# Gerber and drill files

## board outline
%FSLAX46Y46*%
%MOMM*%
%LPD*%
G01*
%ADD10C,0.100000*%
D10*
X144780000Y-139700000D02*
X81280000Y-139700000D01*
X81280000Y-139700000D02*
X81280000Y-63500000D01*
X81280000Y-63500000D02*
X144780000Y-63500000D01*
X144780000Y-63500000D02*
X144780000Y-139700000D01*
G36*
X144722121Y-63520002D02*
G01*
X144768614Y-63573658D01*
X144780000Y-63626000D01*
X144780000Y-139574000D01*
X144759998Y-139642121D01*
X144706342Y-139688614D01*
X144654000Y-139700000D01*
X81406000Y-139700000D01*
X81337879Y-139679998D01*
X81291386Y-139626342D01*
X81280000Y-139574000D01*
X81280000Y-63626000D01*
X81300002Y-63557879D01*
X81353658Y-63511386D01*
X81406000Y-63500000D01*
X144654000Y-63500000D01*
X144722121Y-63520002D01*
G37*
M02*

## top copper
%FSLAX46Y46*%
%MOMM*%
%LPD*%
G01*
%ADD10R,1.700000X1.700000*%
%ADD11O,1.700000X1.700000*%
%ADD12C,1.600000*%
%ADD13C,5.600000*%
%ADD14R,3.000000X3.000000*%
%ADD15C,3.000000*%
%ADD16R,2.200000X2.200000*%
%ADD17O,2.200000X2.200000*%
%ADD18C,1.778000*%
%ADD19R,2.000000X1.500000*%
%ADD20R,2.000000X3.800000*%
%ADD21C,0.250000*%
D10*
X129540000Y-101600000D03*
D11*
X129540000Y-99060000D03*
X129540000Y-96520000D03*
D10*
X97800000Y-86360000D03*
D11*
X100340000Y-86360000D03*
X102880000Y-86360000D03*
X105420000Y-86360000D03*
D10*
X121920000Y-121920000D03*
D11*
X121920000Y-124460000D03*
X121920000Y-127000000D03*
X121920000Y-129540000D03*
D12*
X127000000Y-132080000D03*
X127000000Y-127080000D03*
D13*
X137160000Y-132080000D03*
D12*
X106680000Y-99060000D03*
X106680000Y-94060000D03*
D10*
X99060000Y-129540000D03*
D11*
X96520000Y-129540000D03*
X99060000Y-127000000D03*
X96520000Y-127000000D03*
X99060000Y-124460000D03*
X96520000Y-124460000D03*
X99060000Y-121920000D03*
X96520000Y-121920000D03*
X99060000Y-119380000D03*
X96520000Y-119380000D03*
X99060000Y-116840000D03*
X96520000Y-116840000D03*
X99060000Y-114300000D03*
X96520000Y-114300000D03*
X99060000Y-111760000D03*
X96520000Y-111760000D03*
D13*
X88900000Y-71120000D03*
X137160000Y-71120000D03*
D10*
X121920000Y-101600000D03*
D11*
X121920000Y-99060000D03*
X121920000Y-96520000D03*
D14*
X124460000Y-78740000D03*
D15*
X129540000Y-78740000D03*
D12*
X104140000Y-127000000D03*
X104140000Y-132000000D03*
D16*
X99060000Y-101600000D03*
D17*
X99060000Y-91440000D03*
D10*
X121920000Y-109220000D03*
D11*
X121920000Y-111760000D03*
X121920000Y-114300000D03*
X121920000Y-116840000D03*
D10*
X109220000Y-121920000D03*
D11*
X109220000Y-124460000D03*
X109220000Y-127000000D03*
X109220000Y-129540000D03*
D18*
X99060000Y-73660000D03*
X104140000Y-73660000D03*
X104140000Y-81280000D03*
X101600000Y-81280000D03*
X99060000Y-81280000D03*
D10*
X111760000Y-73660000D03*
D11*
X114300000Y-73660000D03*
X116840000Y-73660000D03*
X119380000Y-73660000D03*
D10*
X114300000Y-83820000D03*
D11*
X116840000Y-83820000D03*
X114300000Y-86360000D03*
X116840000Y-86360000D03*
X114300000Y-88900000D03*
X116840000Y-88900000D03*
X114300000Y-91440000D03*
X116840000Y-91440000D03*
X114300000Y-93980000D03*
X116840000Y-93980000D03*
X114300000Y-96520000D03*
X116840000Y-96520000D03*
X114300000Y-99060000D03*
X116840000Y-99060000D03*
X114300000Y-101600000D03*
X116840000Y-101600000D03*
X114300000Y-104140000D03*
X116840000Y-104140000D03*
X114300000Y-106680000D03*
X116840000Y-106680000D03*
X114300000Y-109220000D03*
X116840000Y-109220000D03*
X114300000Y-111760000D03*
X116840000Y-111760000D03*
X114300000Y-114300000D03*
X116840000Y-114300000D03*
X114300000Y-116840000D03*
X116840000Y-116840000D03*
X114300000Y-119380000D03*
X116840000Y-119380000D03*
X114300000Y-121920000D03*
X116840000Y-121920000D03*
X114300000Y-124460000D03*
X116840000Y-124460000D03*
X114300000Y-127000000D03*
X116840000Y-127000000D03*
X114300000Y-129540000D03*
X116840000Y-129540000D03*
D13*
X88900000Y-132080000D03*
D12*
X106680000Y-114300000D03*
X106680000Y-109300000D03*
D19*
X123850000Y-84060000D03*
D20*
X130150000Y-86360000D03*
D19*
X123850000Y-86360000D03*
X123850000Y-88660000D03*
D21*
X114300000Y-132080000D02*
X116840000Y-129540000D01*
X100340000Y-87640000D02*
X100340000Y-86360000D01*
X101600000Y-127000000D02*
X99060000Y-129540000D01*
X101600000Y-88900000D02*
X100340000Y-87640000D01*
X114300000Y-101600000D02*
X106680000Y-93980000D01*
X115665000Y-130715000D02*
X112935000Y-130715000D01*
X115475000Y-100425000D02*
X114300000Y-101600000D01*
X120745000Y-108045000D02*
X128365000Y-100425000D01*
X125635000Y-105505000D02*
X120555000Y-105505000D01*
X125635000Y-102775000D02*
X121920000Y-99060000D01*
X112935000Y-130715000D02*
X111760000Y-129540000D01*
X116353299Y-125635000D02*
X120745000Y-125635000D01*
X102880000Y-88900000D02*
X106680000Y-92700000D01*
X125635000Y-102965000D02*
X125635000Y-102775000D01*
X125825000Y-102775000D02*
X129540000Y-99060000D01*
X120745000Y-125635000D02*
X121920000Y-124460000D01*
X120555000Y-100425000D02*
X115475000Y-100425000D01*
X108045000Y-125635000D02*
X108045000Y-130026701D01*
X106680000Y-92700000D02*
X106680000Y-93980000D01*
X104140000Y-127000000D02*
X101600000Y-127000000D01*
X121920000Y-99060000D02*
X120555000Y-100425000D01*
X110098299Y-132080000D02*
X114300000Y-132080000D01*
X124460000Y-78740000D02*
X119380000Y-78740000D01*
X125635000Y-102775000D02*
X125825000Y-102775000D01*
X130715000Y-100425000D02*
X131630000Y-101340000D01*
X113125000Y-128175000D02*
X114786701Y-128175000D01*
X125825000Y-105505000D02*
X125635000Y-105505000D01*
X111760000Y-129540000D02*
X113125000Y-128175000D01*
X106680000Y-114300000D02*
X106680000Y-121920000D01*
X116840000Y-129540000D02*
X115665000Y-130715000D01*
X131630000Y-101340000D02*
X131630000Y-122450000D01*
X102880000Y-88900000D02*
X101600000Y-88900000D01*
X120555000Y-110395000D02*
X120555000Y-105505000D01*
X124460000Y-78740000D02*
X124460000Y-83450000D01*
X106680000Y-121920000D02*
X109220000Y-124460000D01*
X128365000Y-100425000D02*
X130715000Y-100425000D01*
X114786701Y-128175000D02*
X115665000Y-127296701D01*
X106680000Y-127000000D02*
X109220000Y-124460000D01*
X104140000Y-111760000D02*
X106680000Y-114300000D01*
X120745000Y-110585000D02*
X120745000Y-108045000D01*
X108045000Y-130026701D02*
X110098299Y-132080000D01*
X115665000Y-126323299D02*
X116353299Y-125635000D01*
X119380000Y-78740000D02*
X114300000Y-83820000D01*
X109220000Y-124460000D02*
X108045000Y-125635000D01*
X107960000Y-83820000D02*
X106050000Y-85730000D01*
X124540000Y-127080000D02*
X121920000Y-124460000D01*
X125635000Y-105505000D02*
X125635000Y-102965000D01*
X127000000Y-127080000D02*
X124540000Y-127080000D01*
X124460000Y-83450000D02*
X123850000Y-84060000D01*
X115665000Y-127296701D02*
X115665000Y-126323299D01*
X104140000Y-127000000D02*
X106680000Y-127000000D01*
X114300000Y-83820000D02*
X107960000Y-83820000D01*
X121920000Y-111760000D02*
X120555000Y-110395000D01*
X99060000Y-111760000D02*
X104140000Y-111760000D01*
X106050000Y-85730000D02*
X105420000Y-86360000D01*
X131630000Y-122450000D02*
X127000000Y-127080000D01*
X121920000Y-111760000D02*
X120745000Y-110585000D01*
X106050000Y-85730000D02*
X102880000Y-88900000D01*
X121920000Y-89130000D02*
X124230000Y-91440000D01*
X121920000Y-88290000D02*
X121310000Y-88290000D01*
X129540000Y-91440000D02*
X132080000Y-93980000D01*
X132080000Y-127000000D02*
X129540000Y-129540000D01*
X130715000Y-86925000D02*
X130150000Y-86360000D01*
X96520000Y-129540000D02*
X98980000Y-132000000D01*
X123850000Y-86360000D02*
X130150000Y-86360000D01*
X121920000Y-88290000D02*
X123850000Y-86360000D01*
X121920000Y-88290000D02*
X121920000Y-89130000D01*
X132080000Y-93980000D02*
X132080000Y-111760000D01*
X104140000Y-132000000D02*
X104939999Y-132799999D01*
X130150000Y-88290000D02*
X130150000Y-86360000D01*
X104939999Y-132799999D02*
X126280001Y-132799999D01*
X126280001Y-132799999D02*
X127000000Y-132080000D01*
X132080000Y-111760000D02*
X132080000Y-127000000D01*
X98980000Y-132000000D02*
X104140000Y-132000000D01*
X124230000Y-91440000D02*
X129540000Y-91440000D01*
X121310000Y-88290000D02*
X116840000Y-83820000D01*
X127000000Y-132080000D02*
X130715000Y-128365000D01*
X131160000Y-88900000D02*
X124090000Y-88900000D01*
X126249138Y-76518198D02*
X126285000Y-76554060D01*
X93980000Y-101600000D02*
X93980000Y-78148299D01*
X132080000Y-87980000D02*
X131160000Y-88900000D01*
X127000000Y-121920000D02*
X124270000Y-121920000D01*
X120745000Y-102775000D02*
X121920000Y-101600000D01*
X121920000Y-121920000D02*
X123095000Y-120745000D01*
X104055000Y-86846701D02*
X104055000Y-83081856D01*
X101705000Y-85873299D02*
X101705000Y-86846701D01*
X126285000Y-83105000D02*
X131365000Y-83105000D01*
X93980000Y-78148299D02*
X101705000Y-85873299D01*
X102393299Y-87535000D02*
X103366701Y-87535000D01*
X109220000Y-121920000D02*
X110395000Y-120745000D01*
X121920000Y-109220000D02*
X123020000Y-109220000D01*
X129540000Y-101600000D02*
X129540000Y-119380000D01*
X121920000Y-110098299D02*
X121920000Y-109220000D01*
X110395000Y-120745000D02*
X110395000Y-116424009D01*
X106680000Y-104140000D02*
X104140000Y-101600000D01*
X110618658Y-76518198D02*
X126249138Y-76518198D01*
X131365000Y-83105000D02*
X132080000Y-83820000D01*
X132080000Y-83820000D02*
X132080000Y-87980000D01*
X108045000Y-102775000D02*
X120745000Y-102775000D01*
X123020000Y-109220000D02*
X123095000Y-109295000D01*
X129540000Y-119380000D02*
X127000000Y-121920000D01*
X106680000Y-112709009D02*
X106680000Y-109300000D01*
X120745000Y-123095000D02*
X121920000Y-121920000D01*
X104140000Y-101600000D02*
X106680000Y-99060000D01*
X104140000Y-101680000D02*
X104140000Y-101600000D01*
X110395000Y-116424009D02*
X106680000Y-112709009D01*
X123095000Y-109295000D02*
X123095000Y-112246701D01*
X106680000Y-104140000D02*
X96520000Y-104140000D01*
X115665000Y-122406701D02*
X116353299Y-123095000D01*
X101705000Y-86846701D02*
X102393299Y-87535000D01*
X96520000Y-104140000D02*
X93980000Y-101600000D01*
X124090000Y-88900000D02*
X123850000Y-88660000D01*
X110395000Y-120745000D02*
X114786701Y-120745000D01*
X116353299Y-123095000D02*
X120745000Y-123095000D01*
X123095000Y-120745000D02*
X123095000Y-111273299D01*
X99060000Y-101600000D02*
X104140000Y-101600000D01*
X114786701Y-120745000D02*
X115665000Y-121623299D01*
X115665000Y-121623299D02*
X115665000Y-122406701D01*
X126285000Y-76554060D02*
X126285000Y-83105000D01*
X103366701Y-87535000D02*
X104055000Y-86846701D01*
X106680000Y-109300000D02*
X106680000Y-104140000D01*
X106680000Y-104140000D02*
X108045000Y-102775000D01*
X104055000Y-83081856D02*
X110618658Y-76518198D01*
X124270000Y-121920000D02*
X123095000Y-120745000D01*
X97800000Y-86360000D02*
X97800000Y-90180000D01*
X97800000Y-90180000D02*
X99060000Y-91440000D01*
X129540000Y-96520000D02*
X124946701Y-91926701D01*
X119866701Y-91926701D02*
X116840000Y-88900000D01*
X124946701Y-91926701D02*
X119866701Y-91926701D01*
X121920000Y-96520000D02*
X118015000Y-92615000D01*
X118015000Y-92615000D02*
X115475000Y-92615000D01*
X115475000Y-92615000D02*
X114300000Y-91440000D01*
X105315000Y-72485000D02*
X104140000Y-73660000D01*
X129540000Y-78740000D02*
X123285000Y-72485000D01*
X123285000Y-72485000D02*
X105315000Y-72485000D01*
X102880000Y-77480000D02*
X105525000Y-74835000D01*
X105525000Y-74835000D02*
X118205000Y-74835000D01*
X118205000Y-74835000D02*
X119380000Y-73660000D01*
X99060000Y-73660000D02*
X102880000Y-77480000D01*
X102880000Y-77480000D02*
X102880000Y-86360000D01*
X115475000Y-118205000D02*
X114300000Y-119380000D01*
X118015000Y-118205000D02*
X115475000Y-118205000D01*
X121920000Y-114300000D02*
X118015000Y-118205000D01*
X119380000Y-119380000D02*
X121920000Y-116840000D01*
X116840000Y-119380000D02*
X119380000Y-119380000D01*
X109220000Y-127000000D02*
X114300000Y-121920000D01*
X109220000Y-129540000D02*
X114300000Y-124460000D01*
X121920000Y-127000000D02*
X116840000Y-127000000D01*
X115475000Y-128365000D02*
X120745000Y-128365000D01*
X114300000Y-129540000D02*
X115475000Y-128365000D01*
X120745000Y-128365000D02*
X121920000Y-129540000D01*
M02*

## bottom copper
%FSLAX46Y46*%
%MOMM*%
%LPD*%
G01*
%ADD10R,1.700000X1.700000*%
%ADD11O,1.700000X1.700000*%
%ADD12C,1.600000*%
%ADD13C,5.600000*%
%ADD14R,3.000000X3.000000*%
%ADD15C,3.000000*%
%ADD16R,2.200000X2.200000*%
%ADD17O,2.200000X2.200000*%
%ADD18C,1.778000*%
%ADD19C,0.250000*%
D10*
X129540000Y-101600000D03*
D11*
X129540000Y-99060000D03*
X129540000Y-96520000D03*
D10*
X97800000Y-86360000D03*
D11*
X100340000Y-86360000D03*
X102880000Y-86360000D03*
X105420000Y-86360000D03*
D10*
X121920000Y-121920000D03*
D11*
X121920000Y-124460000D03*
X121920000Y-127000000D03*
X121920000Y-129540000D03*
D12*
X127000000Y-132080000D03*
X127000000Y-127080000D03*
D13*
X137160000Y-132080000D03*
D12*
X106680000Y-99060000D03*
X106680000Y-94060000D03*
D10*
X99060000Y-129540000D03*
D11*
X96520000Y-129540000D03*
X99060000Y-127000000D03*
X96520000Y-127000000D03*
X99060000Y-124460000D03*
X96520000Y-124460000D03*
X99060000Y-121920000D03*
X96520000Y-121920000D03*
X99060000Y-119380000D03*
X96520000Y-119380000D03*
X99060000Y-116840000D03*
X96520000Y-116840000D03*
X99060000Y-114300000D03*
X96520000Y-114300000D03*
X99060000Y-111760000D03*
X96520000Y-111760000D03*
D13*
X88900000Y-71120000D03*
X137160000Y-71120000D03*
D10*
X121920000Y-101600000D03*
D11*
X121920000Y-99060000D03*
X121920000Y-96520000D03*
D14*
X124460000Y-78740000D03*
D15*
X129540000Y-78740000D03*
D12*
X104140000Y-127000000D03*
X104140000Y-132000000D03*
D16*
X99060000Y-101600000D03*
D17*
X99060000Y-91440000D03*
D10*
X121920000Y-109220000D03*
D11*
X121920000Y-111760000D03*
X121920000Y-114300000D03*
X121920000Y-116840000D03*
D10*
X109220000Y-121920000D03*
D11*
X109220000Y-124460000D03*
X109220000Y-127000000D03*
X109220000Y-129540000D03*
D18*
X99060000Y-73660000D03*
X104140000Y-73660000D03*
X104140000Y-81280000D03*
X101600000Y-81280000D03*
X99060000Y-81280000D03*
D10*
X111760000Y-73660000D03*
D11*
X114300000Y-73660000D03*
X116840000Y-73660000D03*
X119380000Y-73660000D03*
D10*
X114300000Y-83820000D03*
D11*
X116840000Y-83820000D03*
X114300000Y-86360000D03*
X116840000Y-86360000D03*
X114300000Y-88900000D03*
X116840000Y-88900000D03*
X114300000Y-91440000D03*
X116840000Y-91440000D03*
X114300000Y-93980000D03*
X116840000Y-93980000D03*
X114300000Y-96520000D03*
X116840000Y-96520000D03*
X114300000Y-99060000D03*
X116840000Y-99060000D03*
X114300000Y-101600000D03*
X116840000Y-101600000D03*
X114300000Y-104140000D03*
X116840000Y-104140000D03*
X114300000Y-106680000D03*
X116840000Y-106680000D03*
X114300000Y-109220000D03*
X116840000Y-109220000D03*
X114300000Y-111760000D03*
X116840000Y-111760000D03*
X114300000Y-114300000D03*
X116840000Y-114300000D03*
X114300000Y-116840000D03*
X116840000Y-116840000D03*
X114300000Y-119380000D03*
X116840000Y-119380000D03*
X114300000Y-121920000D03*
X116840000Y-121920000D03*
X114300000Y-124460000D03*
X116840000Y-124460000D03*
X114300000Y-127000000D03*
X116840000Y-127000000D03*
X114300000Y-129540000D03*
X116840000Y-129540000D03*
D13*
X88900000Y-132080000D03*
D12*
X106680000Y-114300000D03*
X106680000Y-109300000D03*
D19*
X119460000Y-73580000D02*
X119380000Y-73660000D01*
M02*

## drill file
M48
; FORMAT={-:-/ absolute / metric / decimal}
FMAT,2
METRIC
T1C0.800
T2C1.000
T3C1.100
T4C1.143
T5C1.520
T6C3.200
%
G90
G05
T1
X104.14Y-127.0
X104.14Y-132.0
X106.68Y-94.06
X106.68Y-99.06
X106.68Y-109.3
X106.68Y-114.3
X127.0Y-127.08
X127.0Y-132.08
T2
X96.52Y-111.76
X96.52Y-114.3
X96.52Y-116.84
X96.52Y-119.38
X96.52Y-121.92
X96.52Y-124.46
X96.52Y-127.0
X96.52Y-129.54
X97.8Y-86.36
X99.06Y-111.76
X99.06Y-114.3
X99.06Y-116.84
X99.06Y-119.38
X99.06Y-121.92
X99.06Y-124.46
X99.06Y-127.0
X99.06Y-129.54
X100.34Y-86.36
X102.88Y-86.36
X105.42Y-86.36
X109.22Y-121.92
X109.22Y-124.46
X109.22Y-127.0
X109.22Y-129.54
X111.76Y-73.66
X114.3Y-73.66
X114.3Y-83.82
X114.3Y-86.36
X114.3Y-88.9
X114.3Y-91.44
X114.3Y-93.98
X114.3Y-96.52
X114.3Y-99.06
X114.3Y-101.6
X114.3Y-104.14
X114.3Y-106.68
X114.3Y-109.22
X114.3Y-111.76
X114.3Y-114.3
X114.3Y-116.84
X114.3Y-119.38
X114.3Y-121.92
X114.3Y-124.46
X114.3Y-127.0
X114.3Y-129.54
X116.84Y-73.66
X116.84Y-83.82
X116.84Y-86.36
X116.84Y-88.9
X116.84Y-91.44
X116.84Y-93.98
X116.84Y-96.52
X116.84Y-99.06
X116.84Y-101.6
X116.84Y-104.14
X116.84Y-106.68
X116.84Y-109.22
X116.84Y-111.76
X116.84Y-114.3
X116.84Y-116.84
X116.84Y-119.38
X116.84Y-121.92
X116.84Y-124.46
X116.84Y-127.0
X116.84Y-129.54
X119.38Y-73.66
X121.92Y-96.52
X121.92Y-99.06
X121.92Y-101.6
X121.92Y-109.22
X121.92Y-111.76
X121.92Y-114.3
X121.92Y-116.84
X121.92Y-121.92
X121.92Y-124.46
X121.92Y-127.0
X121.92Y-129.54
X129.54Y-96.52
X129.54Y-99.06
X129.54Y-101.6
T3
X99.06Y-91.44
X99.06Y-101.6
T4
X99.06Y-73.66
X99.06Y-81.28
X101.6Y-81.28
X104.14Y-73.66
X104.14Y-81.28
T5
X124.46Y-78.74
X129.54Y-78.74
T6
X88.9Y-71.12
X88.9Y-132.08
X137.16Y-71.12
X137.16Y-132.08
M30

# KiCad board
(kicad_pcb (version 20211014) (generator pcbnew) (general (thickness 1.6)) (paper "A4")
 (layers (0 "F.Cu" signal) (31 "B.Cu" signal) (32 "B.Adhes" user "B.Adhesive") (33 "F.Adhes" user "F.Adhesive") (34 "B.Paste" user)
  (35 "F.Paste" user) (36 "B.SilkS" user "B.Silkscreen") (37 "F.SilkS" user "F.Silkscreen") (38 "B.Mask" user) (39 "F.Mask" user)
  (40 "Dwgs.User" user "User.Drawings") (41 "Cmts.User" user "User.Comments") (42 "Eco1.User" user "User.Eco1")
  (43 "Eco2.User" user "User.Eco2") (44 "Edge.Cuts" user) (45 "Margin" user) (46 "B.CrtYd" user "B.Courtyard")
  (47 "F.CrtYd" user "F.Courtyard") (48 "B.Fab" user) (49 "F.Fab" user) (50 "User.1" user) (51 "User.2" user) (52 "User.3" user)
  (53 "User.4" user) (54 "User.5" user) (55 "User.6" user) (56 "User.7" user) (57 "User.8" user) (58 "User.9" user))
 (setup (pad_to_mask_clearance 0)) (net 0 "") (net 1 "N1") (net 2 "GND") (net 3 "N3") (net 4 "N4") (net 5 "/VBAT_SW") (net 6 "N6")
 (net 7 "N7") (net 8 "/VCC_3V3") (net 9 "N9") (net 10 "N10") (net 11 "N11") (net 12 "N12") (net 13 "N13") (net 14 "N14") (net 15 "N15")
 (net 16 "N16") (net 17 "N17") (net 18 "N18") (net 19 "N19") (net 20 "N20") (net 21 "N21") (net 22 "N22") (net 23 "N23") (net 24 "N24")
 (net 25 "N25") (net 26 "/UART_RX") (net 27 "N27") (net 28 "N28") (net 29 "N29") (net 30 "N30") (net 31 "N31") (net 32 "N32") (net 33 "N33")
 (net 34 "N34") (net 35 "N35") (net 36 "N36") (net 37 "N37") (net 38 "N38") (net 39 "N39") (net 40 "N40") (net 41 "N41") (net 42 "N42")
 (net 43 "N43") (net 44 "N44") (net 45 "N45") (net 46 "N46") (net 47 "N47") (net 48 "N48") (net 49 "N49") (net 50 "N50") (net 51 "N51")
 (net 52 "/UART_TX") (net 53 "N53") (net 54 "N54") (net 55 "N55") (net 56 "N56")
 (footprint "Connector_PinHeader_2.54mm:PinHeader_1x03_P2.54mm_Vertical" (layer "F.Cu") (at 129.54 101.6 180)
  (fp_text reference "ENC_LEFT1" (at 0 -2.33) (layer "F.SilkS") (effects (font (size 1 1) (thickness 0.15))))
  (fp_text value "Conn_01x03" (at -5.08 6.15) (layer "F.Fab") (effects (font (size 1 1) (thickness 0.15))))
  (pad "1" thru_hole rect (at 0 0 180) (size 1.7 1.7) (drill 1) (layers *.Cu *.Mask) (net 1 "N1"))
  (pad "2" thru_hole oval (at 0 2.54 180) (size 1.7 1.7) (drill 1) (layers *.Cu *.Mask) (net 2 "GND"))
  (pad "3" thru_hole oval (at 0 5.08 180) (size 1.7 1.7) (drill 1) (layers *.Cu *.Mask) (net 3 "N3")))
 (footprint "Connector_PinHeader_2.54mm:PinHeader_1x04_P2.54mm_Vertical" (layer "F.Cu") (at 97.8 86.36 90)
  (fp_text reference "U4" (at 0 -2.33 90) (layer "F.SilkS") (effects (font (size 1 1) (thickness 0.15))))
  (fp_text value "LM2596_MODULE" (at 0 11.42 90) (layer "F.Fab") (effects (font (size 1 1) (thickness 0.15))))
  (pad "1" thru_hole rect (at 0 0 90) (size 1.7 1.7) (drill 1) (layers *.Cu *.Mask) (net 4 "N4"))
  (pad "2" thru_hole oval (at 0 2.54 90) (size 1.7 1.7) (drill 1) (layers *.Cu *.Mask) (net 2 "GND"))
  (pad "3" thru_hole oval (at 0 5.08 90) (size 1.7 1.7) (drill 1) (layers *.Cu *.Mask) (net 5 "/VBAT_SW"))
  (pad "4" thru_hole oval (at 0 7.62 90) (size 1.7 1.7) (drill 1) (layers *.Cu *.Mask) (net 2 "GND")))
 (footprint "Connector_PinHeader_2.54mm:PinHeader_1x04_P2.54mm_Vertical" (layer "F.Cu") (at 121.92 121.92)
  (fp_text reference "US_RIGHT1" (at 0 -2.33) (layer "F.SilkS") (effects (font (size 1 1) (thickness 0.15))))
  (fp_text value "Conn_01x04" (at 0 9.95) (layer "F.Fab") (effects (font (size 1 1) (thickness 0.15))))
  (pad "1" thru_hole rect (at 0 0) (size 1.7 1.7) (drill 1) (layers *.Cu *.Mask) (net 1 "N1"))
  (pad "2" thru_hole oval (at 0 2.54) (size 1.7 1.7) (drill 1) (layers *.Cu *.Mask) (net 2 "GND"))
  (pad "3" thru_hole oval (at 0 5.08) (size 1.7 1.7) (drill 1) (layers *.Cu *.Mask) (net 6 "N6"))
  (pad "4" thru_hole oval (at 0 7.62) (size 1.7 1.7) (drill 1) (layers *.Cu *.Mask) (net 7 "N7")))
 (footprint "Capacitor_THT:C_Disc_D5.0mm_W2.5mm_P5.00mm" (layer "F.Cu") (at 127 132.08 90)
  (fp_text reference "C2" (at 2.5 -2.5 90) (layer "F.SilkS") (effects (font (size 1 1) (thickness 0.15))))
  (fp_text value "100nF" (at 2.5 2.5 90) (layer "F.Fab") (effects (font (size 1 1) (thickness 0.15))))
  (pad "1" thru_hole circle (at 0 0 90) (size 1.6 1.6) (drill 0.8) (layers *.Cu *.Mask) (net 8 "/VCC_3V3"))
  (pad "2" thru_hole circle (at 5 0 90) (size 1.6 1.6) (drill 0.8) (layers *.Cu *.Mask) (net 2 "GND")))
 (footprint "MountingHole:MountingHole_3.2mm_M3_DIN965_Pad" (layer "F.Cu") (at 137.16 132.08)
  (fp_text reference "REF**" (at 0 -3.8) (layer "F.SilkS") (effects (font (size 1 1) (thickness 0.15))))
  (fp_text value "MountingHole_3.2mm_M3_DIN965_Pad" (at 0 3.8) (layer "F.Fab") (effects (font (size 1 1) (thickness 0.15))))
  (pad "1" thru_hole circle (at 0 0) (size 5.6 5.6) (drill 3.2) (layers *.Cu *.Mask)))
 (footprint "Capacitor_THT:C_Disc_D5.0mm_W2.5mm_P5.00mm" (layer "F.Cu") (at 106.68 99.06 90)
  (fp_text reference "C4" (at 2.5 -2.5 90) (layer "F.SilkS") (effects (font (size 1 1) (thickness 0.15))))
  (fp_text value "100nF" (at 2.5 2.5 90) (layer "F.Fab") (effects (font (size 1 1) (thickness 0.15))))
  (pad "1" thru_hole circle (at 0 0 90) (size 1.6 1.6) (drill 0.8) (layers *.Cu *.Mask) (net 1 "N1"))
  (pad "2" thru_hole circle (at 5 0 90) (size 1.6 1.6) (drill 0.8) (layers *.Cu *.Mask) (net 2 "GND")))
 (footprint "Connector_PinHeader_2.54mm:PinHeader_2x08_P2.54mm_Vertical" (layer "F.Cu") (at 99.06 129.54 180)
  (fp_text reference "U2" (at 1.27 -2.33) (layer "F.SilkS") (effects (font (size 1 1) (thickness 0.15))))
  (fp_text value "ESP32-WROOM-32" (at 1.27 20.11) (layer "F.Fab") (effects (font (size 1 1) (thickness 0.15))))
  (pad "1" thru_hole rect (at 0 0 180) (size 1.7 1.7) (drill 1) (layers *.Cu *.Mask) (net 2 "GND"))
  (pad "2" thru_hole oval (at 2.54 0 180) (size 1.7 1.7) (drill 1) (layers *.Cu *.Mask) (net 8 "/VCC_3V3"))
  (pad "3" thru_hole oval (at 0 2.54 180) (size 1.7 1.7) (drill 1) (layers *.Cu *.Mask) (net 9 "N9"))
  (pad "4" thru_hole oval (at 2.54 2.54 180) (size 1.7 1.7) (drill 1) (layers *.Cu *.Mask) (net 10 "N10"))
  (pad "5" thru_hole oval (at 0 5.08 180) (size 1.7 1.7) (drill 1) (layers *.Cu *.Mask) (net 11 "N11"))
  (pad "6" thru_hole oval (at 2.54 5.08 180) (size 1.7 1.7) (drill 1) (layers *.Cu *.Mask) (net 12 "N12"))
  (pad "7" thru_hole oval (at 0 7.62 180) (size 1.7 1.7) (drill 1) (layers *.Cu *.Mask) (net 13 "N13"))
  (pad "8" thru_hole oval (at 2.54 7.62 180) (size 1.7 1.7) (drill 1) (layers *.Cu *.Mask) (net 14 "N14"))
  (pad "9" thru_hole oval (at 0 10.16 180) (size 1.7 1.7) (drill 1) (layers *.Cu *.Mask) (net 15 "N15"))
  (pad "10" thru_hole oval (at 2.54 10.16 180) (size 1.7 1.7) (drill 1) (layers *.Cu *.Mask) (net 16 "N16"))
  (pad "11" thru_hole oval (at 0 12.7 180) (size 1.7 1.7) (drill 1) (layers *.Cu *.Mask) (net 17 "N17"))
  (pad "12" thru_hole oval (at 2.54 12.7 180) (size 1.7 1.7) (drill 1) (layers *.Cu *.Mask) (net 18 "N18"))
  (pad "13" thru_hole oval (at 0 15.24 180) (size 1.7 1.7) (drill 1) (layers *.Cu *.Mask) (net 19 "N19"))
  (pad "14" thru_hole oval (at 2.54 15.24 180) (size 1.7 1.7) (drill 1) (layers *.Cu *.Mask) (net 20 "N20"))
  (pad "15" thru_hole oval (at 0 17.78 180) (size 1.7 1.7) (drill 1) (layers *.Cu *.Mask) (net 2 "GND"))
  (pad "16" thru_hole oval (at 2.54 17.78 180) (size 1.7 1.7) (drill 1) (layers *.Cu *.Mask) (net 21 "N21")))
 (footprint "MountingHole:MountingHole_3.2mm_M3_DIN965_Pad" (layer "F.Cu") (at 88.9 71.12)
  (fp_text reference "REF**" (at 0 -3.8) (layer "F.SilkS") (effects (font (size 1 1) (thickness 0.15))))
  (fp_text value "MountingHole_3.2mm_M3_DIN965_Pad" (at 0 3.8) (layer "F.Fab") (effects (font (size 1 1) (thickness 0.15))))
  (pad "1" thru_hole circle (at 0 0) (size 5.6 5.6) (drill 3.2) (layers *.Cu *.Mask)))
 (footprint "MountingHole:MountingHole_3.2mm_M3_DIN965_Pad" (layer "F.Cu") (at 137.16 71.12)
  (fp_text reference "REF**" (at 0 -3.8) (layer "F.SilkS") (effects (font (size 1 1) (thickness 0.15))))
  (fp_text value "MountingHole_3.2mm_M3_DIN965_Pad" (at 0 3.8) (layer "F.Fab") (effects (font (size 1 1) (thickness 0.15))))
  (pad "1" thru_hole circle (at 0 0) (size 5.6 5.6) (drill 3.2) (layers *.Cu *.Mask)))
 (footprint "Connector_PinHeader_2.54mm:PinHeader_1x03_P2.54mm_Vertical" (layer "F.Cu") (at 121.92 101.6 180)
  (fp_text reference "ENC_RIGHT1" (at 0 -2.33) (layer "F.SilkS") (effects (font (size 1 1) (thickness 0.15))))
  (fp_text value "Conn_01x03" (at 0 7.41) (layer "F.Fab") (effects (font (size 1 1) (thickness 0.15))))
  (pad "1" thru_hole rect (at 0 0 180) (size 1.7 1.7) (drill 1) (layers *.Cu *.Mask) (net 1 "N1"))
  (pad "2" thru_hole oval (at 0 2.54 180) (size 1.7 1.7) (drill 1) (layers *.Cu *.Mask) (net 2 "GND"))
  (pad "3" thru_hole oval (at 0 5.08 180) (size 1.7 1.7) (drill 1) (layers *.Cu *.Mask) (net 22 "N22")))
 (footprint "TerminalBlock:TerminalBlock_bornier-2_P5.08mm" (layer "F.Cu") (at 124.46 78.74)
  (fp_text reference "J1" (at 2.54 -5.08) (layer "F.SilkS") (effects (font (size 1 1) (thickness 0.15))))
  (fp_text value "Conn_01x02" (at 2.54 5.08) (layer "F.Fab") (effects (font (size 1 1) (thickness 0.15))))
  (pad "1" thru_hole rect (at 0 0) (size 3 3) (drill 1.52) (layers *.Cu *.Mask) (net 2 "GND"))
  (pad "2" thru_hole circle (at 5.08 0) (size 3 3) (drill 1.52) (layers *.Cu *.Mask) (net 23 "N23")))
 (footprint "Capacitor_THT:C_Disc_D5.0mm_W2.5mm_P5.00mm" (layer "F.Cu") (at 104.14 127 -90)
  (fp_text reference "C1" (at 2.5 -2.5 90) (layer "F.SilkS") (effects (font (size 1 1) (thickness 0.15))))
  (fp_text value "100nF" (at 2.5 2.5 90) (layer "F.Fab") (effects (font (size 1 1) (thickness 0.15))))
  (pad "1" thru_hole circle (at 0 0 270) (size 1.6 1.6) (drill 0.8) (layers *.Cu *.Mask) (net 2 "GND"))
  (pad "2" thru_hole circle (at 5 0 270) (size 1.6 1.6) (drill 0.8) (layers *.Cu *.Mask) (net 8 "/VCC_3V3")))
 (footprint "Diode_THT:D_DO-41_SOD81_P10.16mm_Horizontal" (layer "F.Cu") (at 99.06 101.6 90)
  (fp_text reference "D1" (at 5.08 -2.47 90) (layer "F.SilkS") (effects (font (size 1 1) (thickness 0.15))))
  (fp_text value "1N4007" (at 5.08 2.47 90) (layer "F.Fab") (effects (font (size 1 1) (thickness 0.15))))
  (pad "1" thru_hole rect (at 0 0 90) (size 2.2 2.2) (drill 1.1) (layers *.Cu *.Mask) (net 1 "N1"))
  (pad "2" thru_hole oval (at 10.16 0 90) (size 2.2 2.2) (drill 1.1) (layers *.Cu *.Mask) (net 4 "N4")))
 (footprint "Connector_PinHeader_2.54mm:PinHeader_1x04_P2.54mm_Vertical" (layer "F.Cu") (at 121.92 109.22)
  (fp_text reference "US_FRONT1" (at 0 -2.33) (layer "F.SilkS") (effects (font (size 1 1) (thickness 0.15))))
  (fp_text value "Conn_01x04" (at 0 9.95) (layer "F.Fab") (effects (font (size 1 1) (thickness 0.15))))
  (pad "1" thru_hole rect (at 0 0) (size 1.7 1.7) (drill 1) (layers *.Cu *.Mask) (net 1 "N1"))
  (pad "2" thru_hole oval (at 0 2.54) (size 1.7 1.7) (drill 1) (layers *.Cu *.Mask) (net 2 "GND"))
  (pad "3" thru_hole oval (at 0 5.08) (size 1.7 1.7) (drill 1) (layers *.Cu *.Mask) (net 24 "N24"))
  (pad "4" thru_hole oval (at 0 7.62) (size 1.7 1.7) (drill 1) (layers *.Cu *.Mask) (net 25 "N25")))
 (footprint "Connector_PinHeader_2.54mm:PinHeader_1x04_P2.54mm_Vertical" (layer "F.Cu") (at 109.22 121.92)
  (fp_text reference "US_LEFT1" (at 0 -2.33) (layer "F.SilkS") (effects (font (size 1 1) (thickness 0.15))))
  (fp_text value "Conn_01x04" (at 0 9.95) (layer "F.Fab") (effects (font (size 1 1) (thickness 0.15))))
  (pad "1" thru_hole rect (at 0 0) (size 1.7 1.7) (drill 1) (layers *.Cu *.Mask) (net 1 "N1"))
  (pad "2" thru_hole oval (at 0 2.54) (size 1.7 1.7) (drill 1) (layers *.Cu *.Mask) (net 2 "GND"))
  (pad "3" thru_hole oval (at 0 5.08) (size 1.7 1.7) (drill 1) (layers *.Cu *.Mask) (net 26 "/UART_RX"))
  (pad "4" thru_hole oval (at 0 7.62) (size 1.7 1.7) (drill 1) (layers *.Cu *.Mask) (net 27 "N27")))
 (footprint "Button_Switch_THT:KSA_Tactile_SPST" (layer "F.Cu") (at 99.06 73.66)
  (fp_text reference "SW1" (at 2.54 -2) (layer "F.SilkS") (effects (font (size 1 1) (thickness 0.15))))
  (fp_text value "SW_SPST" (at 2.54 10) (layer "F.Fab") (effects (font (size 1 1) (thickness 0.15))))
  (pad "1" thru_hole circle (at 0 0) (size 1.778 1.778) (drill 1.143) (layers *.Cu *.Mask) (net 5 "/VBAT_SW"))
  (pad "2" thru_hole circle (at 5.08 0) (size 1.778 1.778) (drill 1.143) (layers *.Cu *.Mask) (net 23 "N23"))
  (pad "3" thru_hole circle (at 5.08 7.62) (size 1.778 1.778) (drill 1.143) (layers *.Cu *.Mask))
  (pad "4" thru_hole circle (at 2.54 7.62) (size 1.778 1.778) (drill 1.143) (layers *.Cu *.Mask))
  (pad "5" thru_hole circle (at 0 7.62) (size 1.778 1.778) (drill 1.143) (layers *.Cu *.Mask)))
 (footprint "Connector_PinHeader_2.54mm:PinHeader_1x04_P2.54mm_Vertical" (layer "F.Cu") (at 111.76 73.66 90)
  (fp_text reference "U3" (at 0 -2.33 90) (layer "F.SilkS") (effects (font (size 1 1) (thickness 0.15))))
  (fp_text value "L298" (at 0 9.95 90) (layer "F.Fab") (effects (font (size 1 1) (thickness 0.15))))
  (pad "1" thru_hole rect (at 0 0 90) (size 1.7 1.7) (drill 1) (layers *.Cu *.Mask) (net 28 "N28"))
  (pad "2" thru_hole oval (at 0 2.54 90) (size 1.7 1.7) (drill 1) (layers *.Cu *.Mask) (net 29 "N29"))
  (pad "3" thru_hole oval (at 0 5.08 90) (size 1.7 1.7) (drill 1) (layers *.Cu *.Mask) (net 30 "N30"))
  (pad "4" thru_hole oval (at 0 7.62 90) (size 1.7 1.7) (drill 1) (layers *.Cu *.Mask) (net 5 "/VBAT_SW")))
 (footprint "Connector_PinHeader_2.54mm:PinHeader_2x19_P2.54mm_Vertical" (layer "F.Cu") (at 114.3 83.82)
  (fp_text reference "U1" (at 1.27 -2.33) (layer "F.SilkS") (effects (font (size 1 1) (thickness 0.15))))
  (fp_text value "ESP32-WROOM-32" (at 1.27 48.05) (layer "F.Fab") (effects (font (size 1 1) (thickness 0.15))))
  (pad "1" thru_hole rect (at 0 0) (size 1.7 1.7) (drill 1) (layers *.Cu *.Mask) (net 2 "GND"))
  (pad "2" thru_hole oval (at 2.54 0) (size 1.7 1.7) (drill 1) (layers *.Cu *.Mask) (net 8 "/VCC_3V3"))
  (pad "3" thru_hole oval (at 0 2.54) (size 1.7 1.7) (drill 1) (layers *.Cu *.Mask) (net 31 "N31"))
  (pad "4" thru_hole oval (at 2.54 2.54) (size 1.7 1.7) (drill 1) (layers *.Cu *.Mask) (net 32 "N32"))
  (pad "5" thru_hole oval (at 0 5.08) (size 1.7 1.7) (drill 1) (layers *.Cu *.Mask) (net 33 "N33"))
  (pad "6" thru_hole oval (at 2.54 5.08) (size 1.7 1.7) (drill 1) (layers *.Cu *.Mask) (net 3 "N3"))
  (pad "7" thru_hole oval (at 0 7.62) (size 1.7 1.7) (drill 1) (layers *.Cu *.Mask) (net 22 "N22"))
  (pad "8" thru_hole oval (at 2.54 7.62) (size 1.7 1.7) (drill 1) (layers *.Cu *.Mask) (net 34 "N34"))
  (pad "9" thru_hole oval (at 0 10.16) (size 1.7 1.7) (drill 1) (layers *.Cu *.Mask) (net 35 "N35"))
  (pad "10" thru_hole oval (at 2.54 10.16) (size 1.7 1.7) (drill 1) (layers *.Cu *.Mask) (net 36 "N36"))
  (pad "11" thru_hole oval (at 0 12.7) (size 1.7 1.7) (drill 1) (layers *.Cu *.Mask) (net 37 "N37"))
  (pad "12" thru_hole oval (at 2.54 12.7) (size 1.7 1.7) (drill 1) (layers *.Cu *.Mask) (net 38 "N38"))
  (pad "13" thru_hole oval (at 0 15.24) (size 1.7 1.7) (drill 1) (layers *.Cu *.Mask) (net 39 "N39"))
  (pad "14" thru_hole oval (at 2.54 15.24) (size 1.7 1.7) (drill 1) (layers *.Cu *.Mask) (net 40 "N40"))
  (pad "15" thru_hole oval (at 0 17.78) (size 1.7 1.7) (drill 1) (layers *.Cu *.Mask) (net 2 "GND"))
  (pad "16" thru_hole oval (at 2.54 17.78) (size 1.7 1.7) (drill 1) (layers *.Cu *.Mask) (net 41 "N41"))
  (pad "17" thru_hole oval (at 0 20.32) (size 1.7 1.7) (drill 1) (layers *.Cu *.Mask) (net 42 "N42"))
  (pad "18" thru_hole oval (at 2.54 20.32) (size 1.7 1.7) (drill 1) (layers *.Cu *.Mask) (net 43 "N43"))
  (pad "19" thru_hole oval (at 0 22.86) (size 1.7 1.7) (drill 1) (layers *.Cu *.Mask) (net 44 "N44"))
  (pad "20" thru_hole oval (at 2.54 22.86) (size 1.7 1.7) (drill 1) (layers *.Cu *.Mask) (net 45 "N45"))
  (pad "21" thru_hole oval (at 0 25.4) (size 1.7 1.7) (drill 1) (layers *.Cu *.Mask) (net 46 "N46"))
  (pad "22" thru_hole oval (at 2.54 25.4) (size 1.7 1.7) (drill 1) (layers *.Cu *.Mask) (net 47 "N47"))
  (pad "23" thru_hole oval (at 0 27.94) (size 1.7 1.7) (drill 1) (layers *.Cu *.Mask) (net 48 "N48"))
  (pad "24" thru_hole oval (at 2.54 27.94) (size 1.7 1.7) (drill 1) (layers *.Cu *.Mask) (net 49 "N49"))
  (pad "25" thru_hole oval (at 0 30.48) (size 1.7 1.7) (drill 1) (layers *.Cu *.Mask) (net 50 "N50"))
  (pad "26" thru_hole oval (at 2.54 30.48) (size 1.7 1.7) (drill 1) (layers *.Cu *.Mask) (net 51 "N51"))
  (pad "27" thru_hole oval (at 0 33.02) (size 1.7 1.7) (drill 1) (layers *.Cu *.Mask) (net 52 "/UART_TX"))
  (pad "28" thru_hole oval (at 2.54 33.02) (size 1.7 1.7) (drill 1) (layers *.Cu *.Mask) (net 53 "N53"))
  (pad "29" thru_hole oval (at 0 35.56) (size 1.7 1.7) (drill 1) (layers *.Cu *.Mask) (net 24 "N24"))
  (pad "30" thru_hole oval (at 2.54 35.56) (size 1.7 1.7) (drill 1) (layers *.Cu *.Mask) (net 25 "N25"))
  (pad "31" thru_hole oval (at 0 38.1) (size 1.7 1.7) (drill 1) (layers *.Cu *.Mask) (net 26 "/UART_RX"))
  (pad "32" thru_hole oval (at 2.54 38.1) (size 1.7 1.7) (drill 1) (layers *.Cu *.Mask) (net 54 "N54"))
  (pad "33" thru_hole oval (at 0 40.64) (size 1.7 1.7) (drill 1) (layers *.Cu *.Mask) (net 27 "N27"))
  (pad "34" thru_hole oval (at 2.54 40.64) (size 1.7 1.7) (drill 1) (layers *.Cu *.Mask) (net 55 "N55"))
  (pad "35" thru_hole oval (at 0 43.18) (size 1.7 1.7) (drill 1) (layers *.Cu *.Mask) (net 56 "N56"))
  (pad "36" thru_hole oval (at 2.54 43.18) (size 1.7 1.7) (drill 1) (layers *.Cu *.Mask) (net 6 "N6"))
  (pad "37" thru_hole oval (at 0 45.72) (size 1.7 1.7) (drill 1) (layers *.Cu *.Mask) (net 7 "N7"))
  (pad "38" thru_hole oval (at 2.54 45.72) (size 1.7 1.7) (drill 1) (layers *.Cu *.Mask) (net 2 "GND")))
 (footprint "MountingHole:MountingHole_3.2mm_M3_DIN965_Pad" (layer "F.Cu") (at 88.9 132.08)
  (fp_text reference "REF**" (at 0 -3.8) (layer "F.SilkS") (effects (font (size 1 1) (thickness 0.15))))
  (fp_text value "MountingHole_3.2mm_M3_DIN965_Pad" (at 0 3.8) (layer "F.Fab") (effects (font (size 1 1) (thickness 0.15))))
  (pad "1" thru_hole circle (at 0 0) (size 5.6 5.6) (drill 3.2) (layers *.Cu *.Mask)))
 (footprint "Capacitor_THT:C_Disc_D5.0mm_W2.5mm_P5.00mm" (layer "F.Cu") (at 106.68 114.3 90)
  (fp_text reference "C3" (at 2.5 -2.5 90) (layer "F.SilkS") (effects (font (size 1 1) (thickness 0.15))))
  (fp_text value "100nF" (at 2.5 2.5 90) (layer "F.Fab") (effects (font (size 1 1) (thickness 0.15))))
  (pad "1" thru_hole circle (at 0 0 90) (size 1.6 1.6) (drill 0.8) (layers *.Cu *.Mask) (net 2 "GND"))
  (pad "2" thru_hole circle (at 5 0 90) (size 1.6 1.6) (drill 0.8) (layers *.Cu *.Mask) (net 1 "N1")))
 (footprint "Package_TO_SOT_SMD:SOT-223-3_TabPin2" (layer "F.Cu") (at 127 86.36)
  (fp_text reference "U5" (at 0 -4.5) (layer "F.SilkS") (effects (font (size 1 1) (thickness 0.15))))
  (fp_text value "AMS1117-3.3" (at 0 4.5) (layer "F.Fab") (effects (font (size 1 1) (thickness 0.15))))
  (pad "1" smd rect (at -3.15 -2.3) (size 2 1.5) (layers "F.Cu" "F.Paste" "F.Mask") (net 2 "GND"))
  (pad "2" smd rect (at 3.15 0) (size 2 3.8) (layers "F.Cu" "F.Paste" "F.Mask") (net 8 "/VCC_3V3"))
  (pad "2" smd rect (at -3.15 0) (size 2 1.5) (layers "F.Cu" "F.Paste" "F.Mask") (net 8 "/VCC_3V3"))
  (pad "3" smd rect (at -3.15 2.3) (size 2 1.5) (layers "F.Cu" "F.Paste" "F.Mask") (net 1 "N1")))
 (gr_line (start 144.78 139.7) (end 81.28 139.7) (layer "Edge.Cuts") (width 0.1))
 (gr_line (start 81.28 139.7) (end 81.28 63.5) (layer "Edge.Cuts") (width 0.1))
 (gr_line (start 81.28 63.5) (end 144.78 63.5) (layer "Edge.Cuts") (width 0.1))
 (gr_line (start 144.78 63.5) (end 144.78 139.7) (layer "Edge.Cuts") (width 0.1))
 (segment (start 114.3 132.08) (end 116.84 129.54) (width 0.25) (layer "F.Cu") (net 2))
 (segment (start 100.34 87.64) (end 100.34 86.36) (width 0.25) (layer "F.Cu") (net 2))
 (segment (start 101.6 127) (end 99.06 129.54) (width 0.25) (layer "F.Cu") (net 2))
 (segment (start 101.6 88.9) (end 100.34 87.64) (width 0.25) (layer "F.Cu") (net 2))
 (segment (start 114.3 101.6) (end 106.68 93.98) (width 0.25) (layer "F.Cu") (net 2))
 (segment (start 115.665 130.715) (end 112.935 130.715) (width 0.25) (layer "F.Cu") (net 2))
 (segment (start 115.475 100.425) (end 114.3 101.6) (width 0.25) (layer "F.Cu") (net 2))
 (segment (start 120.745 108.045) (end 128.365 100.425) (width 0.25) (layer "F.Cu") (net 2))
 (segment (start 125.635 105.505) (end 120.555 105.505) (width 0.25) (layer "F.Cu") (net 2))
 (segment (start 125.635 102.775) (end 121.92 99.06) (width 0.25) (layer "F.Cu") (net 2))
 (segment (start 112.935 130.715) (end 111.76 129.54) (width 0.25) (layer "F.Cu") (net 2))
 (segment (start 116.353299 125.635) (end 120.745 125.635) (width 0.25) (layer "F.Cu") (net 2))
 (segment (start 102.88 88.9) (end 106.68 92.7) (width 0.25) (layer "F.Cu") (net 2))
 (segment (start 125.635 102.965) (end 125.635 102.775) (width 0.25) (layer "F.Cu") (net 2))
 (segment (start 125.825 102.775) (end 129.54 99.06) (width 0.25) (layer "F.Cu") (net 2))
 (segment (start 120.745 125.635) (end 121.92 124.46) (width 0.25) (layer "F.Cu") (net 2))
 (segment (start 120.555 100.425) (end 115.475 100.425) (width 0.25) (layer "F.Cu") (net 2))
 (segment (start 108.045 125.635) (end 108.045 130.026701) (width 0.25) (layer "F.Cu") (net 2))
 (segment (start 106.68 92.7) (end 106.68 93.98) (width 0.25) (layer "F.Cu") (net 2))
 (segment (start 104.14 127) (end 101.6 127) (width 0.25) (layer "F.Cu") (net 2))
 (segment (start 121.92 99.06) (end 120.555 100.425) (width 0.25) (layer "F.Cu") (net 2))
 (segment (start 110.098299 132.08) (end 114.3 132.08) (width 0.25) (layer "F.Cu") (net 2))
 (segment (start 124.46 78.74) (end 119.38 78.74) (width 0.25) (layer "F.Cu") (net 2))
 (segment (start 125.635 102.775) (end 125.825 102.775) (width 0.25) (layer "F.Cu") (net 2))
 (segment (start 130.715 100.425) (end 131.63 101.34) (width 0.25) (layer "F.Cu") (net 2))
 (segment (start 113.125 128.175) (end 114.786701 128.175) (width 0.25) (layer "F.Cu") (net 2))
 (segment (start 125.825 105.505) (end 125.635 105.505) (width 0.25) (layer "F.Cu") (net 2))
 (segment (start 111.76 129.54) (end 113.125 128.175) (width 0.25) (layer "F.Cu") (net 2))
 (segment (start 106.68 114.3) (end 106.68 121.92) (width 0.25) (layer "F.Cu") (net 2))
 (segment (start 116.84 129.54) (end 115.665 130.715) (width 0.25) (layer "F.Cu") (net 2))
 (segment (start 131.63 101.34) (end 131.63 122.45) (width 0.25) (layer "F.Cu") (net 2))
 (segment (start 102.88 88.9) (end 101.6 88.9) (width 0.25) (layer "F.Cu") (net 2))
 (segment (start 120.555 110.395) (end 120.555 105.505) (width 0.25) (layer "F.Cu") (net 2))
 (segment (start 124.46 78.74) (end 124.46 83.45) (width 0.25) (layer "F.Cu") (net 2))
 (segment (start 106.68 121.92) (end 109.22 124.46) (width 0.25) (layer "F.Cu") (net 2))
 (segment (start 128.365 100.425) (end 130.715 100.425) (width 0.25) (layer "F.Cu") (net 2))
 (segment (start 114.786701 128.175) (end 115.665 127.296701) (width 0.25) (layer "F.Cu") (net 2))
 (segment (start 106.68 127) (end 109.22 124.46) (width 0.25) (layer "F.Cu") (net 2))
 (segment (start 104.14 111.76) (end 106.68 114.3) (width 0.25) (layer "F.Cu") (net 2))
 (segment (start 120.745 110.585) (end 120.745 108.045) (width 0.25) (layer "F.Cu") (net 2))
 (segment (start 108.045 130.026701) (end 110.098299 132.08) (width 0.25) (layer "F.Cu") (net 2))
 (segment (start 115.665 126.323299) (end 116.353299 125.635) (width 0.25) (layer "F.Cu") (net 2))
 (segment (start 119.38 78.74) (end 114.3 83.82) (width 0.25) (layer "F.Cu") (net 2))
 (segment (start 109.22 124.46) (end 108.045 125.635) (width 0.25) (layer "F.Cu") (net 2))
 (segment (start 107.96 83.82) (end 106.05 85.73) (width 0.25) (layer "F.Cu") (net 2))
 (segment (start 124.54 127.08) (end 121.92 124.46) (width 0.25) (layer "F.Cu") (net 2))
 (segment (start 125.635 105.505) (end 125.635 102.965) (width 0.25) (layer "F.Cu") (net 2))
 (segment (start 127 127.08) (end 124.54 127.08) (width 0.25) (layer "F.Cu") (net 2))
 (segment (start 124.46 83.45) (end 123.85 84.06) (width 0.25) (layer "F.Cu") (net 2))
 (segment (start 115.665 127.296701) (end 115.665 126.323299) (width 0.25) (layer "F.Cu") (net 2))
 (segment (start 104.14 127) (end 106.68 127) (width 0.25) (layer "F.Cu") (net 2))
 (segment (start 114.3 83.82) (end 107.96 83.82) (width 0.25) (layer "F.Cu") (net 2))
 (segment (start 121.92 111.76) (end 120.555 110.395) (width 0.25) (layer "F.Cu") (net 2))
 (segment (start 99.06 111.76) (end 104.14 111.76) (width 0.25) (layer "F.Cu") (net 2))
 (segment (start 106.05 85.73) (end 105.42 86.36) (width 0.25) (layer "F.Cu") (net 2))
 (segment (start 131.63 122.45) (end 127 127.08) (width 0.25) (layer "F.Cu") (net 2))
 (segment (start 121.92 111.76) (end 120.745 110.585) (width 0.25) (layer "F.Cu") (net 2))
 (segment (start 106.05 85.73) (end 102.88 88.9) (width 0.25) (layer "F.Cu") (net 2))
 (segment (start 121.92 89.13) (end 124.23 91.44) (width 0.25) (layer "F.Cu") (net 8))
 (segment (start 121.92 88.29) (end 121.31 88.29) (width 0.25) (layer "F.Cu") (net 8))
 (segment (start 129.54 91.44) (end 132.08 93.98) (width 0.25) (layer "F.Cu") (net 8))
 (segment (start 132.08 127) (end 129.54 129.54) (width 0.25) (layer "F.Cu") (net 8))
 (segment (start 130.715 86.925) (end 130.15 86.36) (width 0.25) (layer "F.Cu") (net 8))
 (segment (start 96.52 129.54) (end 98.98 132) (width 0.25) (layer "F.Cu") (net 8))
 (segment (start 123.85 86.36) (end 130.15 86.36) (width 0.25) (layer "F.Cu") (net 8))
 (segment (start 121.92 88.29) (end 123.85 86.36) (width 0.25) (layer "F.Cu") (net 8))
 (segment (start 121.92 88.29) (end 121.92 89.13) (width 0.25) (layer "F.Cu") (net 8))
 (segment (start 132.08 93.98) (end 132.08 111.76) (width 0.25) (layer "F.Cu") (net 8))
 (segment (start 104.14 132) (end 104.939999 132.799999) (width 0.25) (layer "F.Cu") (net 8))
 (segment (start 130.15 88.29) (end 130.15 86.36) (width 0.25) (layer "F.Cu") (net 8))
 (segment (start 104.939999 132.799999) (end 126.280001 132.799999) (width 0.25) (layer "F.Cu") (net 8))
 (segment (start 126.280001 132.799999) (end 127 132.08) (width 0.25) (layer "F.Cu") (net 8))
 (segment (start 132.08 111.76) (end 132.08 127) (width 0.25) (layer "F.Cu") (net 8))
 (segment (start 98.98 132) (end 104.14 132) (width 0.25) (layer "F.Cu") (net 8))
 (segment (start 124.23 91.44) (end 129.54 91.44) (width 0.25) (layer "F.Cu") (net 8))
 (segment (start 121.31 88.29) (end 116.84 83.82) (width 0.25) (layer "F.Cu") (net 8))
 (segment (start 127 132.08) (end 130.715 128.365) (width 0.25) (layer "F.Cu") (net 8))
 (segment (start 131.16 88.9) (end 124.09 88.9) (width 0.25) (layer "F.Cu") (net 1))
 (segment (start 126.249138 76.518198) (end 126.285 76.55406) (width 0.25) (layer "F.Cu") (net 1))
 (segment (start 93.98 101.6) (end 93.98 78.148299) (width 0.25) (layer "F.Cu") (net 1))
 (segment (start 132.08 87.98) (end 131.16 88.9) (width 0.25) (layer "F.Cu") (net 1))
 (segment (start 127 121.92) (end 124.27 121.92) (width 0.25) (layer "F.Cu") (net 1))
 (segment (start 120.745 102.775) (end 121.92 101.6) (width 0.25) (layer "F.Cu") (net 1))
 (segment (start 121.92 121.92) (end 123.095 120.745) (width 0.25) (layer "F.Cu") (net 1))
 (segment (start 104.055 86.846701) (end 104.055 83.081856) (width 0.25) (layer "F.Cu") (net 1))
 (segment (start 101.705 85.873299) (end 101.705 86.846701) (width 0.25) (layer "F.Cu") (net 1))
 (segment (start 126.285 83.105) (end 131.365 83.105) (width 0.25) (layer "F.Cu") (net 1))
 (segment (start 93.98 78.148299) (end 101.705 85.873299) (width 0.25) (layer "F.Cu") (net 1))
 (segment (start 102.393299 87.535) (end 103.366701 87.535) (width 0.25) (layer "F.Cu") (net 1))
 (segment (start 109.22 121.92) (end 110.395 120.745) (width 0.25) (layer "F.Cu") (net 1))
 (segment (start 121.92 109.22) (end 123.02 109.22) (width 0.25) (layer "F.Cu") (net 1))
 (segment (start 129.54 101.6) (end 129.54 119.38) (width 0.25) (layer "F.Cu") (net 1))
 (segment (start 121.92 110.098299) (end 121.92 109.22) (width 0.25) (layer "F.Cu") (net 1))
 (segment (start 110.395 120.745) (end 110.395 116.424009) (width 0.25) (layer "F.Cu") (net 1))
 (segment (start 106.68 104.14) (end 104.14 101.6) (width 0.25) (layer "F.Cu") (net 1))
 (segment (start 110.618658 76.518198) (end 126.249138 76.518198) (width 0.25) (layer "F.Cu") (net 1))
 (segment (start 131.365 83.105) (end 132.08 83.82) (width 0.25) (layer "F.Cu") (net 1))
 (segment (start 132.08 83.82) (end 132.08 87.98) (width 0.25) (layer "F.Cu") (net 1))
 (segment (start 108.045 102.775) (end 120.745 102.775) (width 0.25) (layer "F.Cu") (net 1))
 (segment (start 123.02 109.22) (end 123.095 109.295) (width 0.25) (layer "F.Cu") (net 1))
 (segment (start 129.54 119.38) (end 127 121.92) (width 0.25) (layer "F.Cu") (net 1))
 (segment (start 106.68 112.709009) (end 106.68 109.3) (width 0.25) (layer "F.Cu") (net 1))
 (segment (start 120.745 123.095) (end 121.92 121.92) (width 0.25) (layer "F.Cu") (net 1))
 (segment (start 104.14 101.6) (end 106.68 99.06) (width 0.25) (layer "F.Cu") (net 1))
 (segment (start 104.14 101.68) (end 104.14 101.6) (width 0.25) (layer "F.Cu") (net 1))
 (segment (start 110.395 116.424009) (end 106.68 112.709009) (width 0.25) (layer "F.Cu") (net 1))
 (segment (start 123.095 109.295) (end 123.095 112.246701) (width 0.25) (layer "F.Cu") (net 1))
 (segment (start 106.68 104.14) (end 96.52 104.14) (width 0.25) (layer "F.Cu") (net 1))
 (segment (start 115.665 122.406701) (end 116.353299 123.095) (width 0.25) (layer "F.Cu") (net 1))
 (segment (start 101.705 86.846701) (end 102.393299 87.535) (width 0.25) (layer "F.Cu") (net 1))
 (segment (start 96.52 104.14) (end 93.98 101.6) (width 0.25) (layer "F.Cu") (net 1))
 (segment (start 124.09 88.9) (end 123.85 88.66) (width 0.25) (layer "F.Cu") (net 1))
 (segment (start 110.395 120.745) (end 114.786701 120.745) (width 0.25) (layer "F.Cu") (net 1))
 (segment (start 116.353299 123.095) (end 120.745 123.095) (width 0.25) (layer "F.Cu") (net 1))
 (segment (start 123.095 120.745) (end 123.095 111.273299) (width 0.25) (layer "F.Cu") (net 1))
 (segment (start 99.06 101.6) (end 104.14 101.6) (width 0.25) (layer "F.Cu") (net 1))
 (segment (start 114.786701 120.745) (end 115.665 121.623299) (width 0.25) (layer "F.Cu") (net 1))
 (segment (start 115.665 121.623299) (end 115.665 122.406701) (width 0.25) (layer "F.Cu") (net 1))
 (segment (start 126.285 76.55406) (end 126.285 83.105) (width 0.25) (layer "F.Cu") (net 1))
 (segment (start 103.366701 87.535) (end 104.055 86.846701) (width 0.25) (layer "F.Cu") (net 1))
 (segment (start 106.68 109.3) (end 106.68 104.14) (width 0.25) (layer "F.Cu") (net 1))
 (segment (start 106.68 104.14) (end 108.045 102.775) (width 0.25) (layer "F.Cu") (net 1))
 (segment (start 104.055 83.081856) (end 110.618658 76.518198) (width 0.25) (layer "F.Cu") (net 1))
 (segment (start 124.27 121.92) (end 123.095 120.745) (width 0.25) (layer "F.Cu") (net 1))
 (segment (start 97.8 86.36) (end 97.8 90.18) (width 0.25) (layer "F.Cu") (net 4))
 (segment (start 97.8 90.18) (end 99.06 91.44) (width 0.25) (layer "F.Cu") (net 4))
 (segment (start 129.54 96.52) (end 124.946701 91.926701) (width 0.25) (layer "F.Cu") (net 3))
 (segment (start 119.866701 91.926701) (end 116.84 88.9) (width 0.25) (layer "F.Cu") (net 3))
 (segment (start 124.946701 91.926701) (end 119.866701 91.926701) (width 0.25) (layer "F.Cu") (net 3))
 (segment (start 121.92 96.52) (end 118.015 92.615) (width 0.25) (layer "F.Cu") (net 22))
 (segment (start 118.015 92.615) (end 115.475 92.615) (width 0.25) (layer "F.Cu") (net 22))
 (segment (start 115.475 92.615) (end 114.3 91.44) (width 0.25) (layer "F.Cu") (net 22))
 (segment (start 105.315 72.485) (end 104.14 73.66) (width 0.25) (layer "F.Cu") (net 23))
 (segment (start 129.54 78.74) (end 123.285 72.485) (width 0.25) (layer "F.Cu") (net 23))
 (segment (start 123.285 72.485) (end 105.315 72.485) (width 0.25) (layer "F.Cu") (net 23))
 (segment (start 102.88 77.48) (end 105.525 74.835) (width 0.25) (layer "F.Cu") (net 5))
 (segment (start 105.525 74.835) (end 118.205 74.835) (width 0.25) (layer "F.Cu") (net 5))
 (segment (start 118.205 74.835) (end 119.38 73.66) (width 0.25) (layer "F.Cu") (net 5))
 (segment (start 99.06 73.66) (end 102.88 77.48) (width 0.25) (layer "F.Cu") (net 5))
 (segment (start 102.88 77.48) (end 102.88 86.36) (width 0.25) (layer "F.Cu") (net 5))
 (segment (start 119.46 73.58) (end 119.38 73.66) (width 0.25) (layer "B.Cu") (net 5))
 (segment (start 115.475 118.205) (end 114.3 119.38) (width 0.25) (layer "F.Cu") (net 24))
 (segment (start 118.015 118.205) (end 115.475 118.205) (width 0.25) (layer "F.Cu") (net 24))
 (segment (start 121.92 114.3) (end 118.015 118.205) (width 0.25) (layer "F.Cu") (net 24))
 (segment (start 119.38 119.38) (end 121.92 116.84) (width 0.25) (layer "F.Cu") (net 25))
 (segment (start 116.84 119.38) (end 119.38 119.38) (width 0.25) (layer "F.Cu") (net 25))
 (segment (start 109.22 127) (end 114.3 121.92) (width 0.25) (layer "F.Cu") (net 26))
 (segment (start 109.22 129.54) (end 114.3 124.46) (width 0.25) (layer "F.Cu") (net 27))
 (segment (start 121.92 127) (end 116.84 127) (width 0.25) (layer "F.Cu") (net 6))
 (segment (start 115.475 128.365) (end 120.745 128.365) (width 0.25) (layer "F.Cu") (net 7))
 (segment (start 114.3 129.54) (end 115.475 128.365) (width 0.25) (layer "F.Cu") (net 7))
 (segment (start 120.745 128.365) (end 121.92 129.54) (width 0.25) (layer "F.Cu") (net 7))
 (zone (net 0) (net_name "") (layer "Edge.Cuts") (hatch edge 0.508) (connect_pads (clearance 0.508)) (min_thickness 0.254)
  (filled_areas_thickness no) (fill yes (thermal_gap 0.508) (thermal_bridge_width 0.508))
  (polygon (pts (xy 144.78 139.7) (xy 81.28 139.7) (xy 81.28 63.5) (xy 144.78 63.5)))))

